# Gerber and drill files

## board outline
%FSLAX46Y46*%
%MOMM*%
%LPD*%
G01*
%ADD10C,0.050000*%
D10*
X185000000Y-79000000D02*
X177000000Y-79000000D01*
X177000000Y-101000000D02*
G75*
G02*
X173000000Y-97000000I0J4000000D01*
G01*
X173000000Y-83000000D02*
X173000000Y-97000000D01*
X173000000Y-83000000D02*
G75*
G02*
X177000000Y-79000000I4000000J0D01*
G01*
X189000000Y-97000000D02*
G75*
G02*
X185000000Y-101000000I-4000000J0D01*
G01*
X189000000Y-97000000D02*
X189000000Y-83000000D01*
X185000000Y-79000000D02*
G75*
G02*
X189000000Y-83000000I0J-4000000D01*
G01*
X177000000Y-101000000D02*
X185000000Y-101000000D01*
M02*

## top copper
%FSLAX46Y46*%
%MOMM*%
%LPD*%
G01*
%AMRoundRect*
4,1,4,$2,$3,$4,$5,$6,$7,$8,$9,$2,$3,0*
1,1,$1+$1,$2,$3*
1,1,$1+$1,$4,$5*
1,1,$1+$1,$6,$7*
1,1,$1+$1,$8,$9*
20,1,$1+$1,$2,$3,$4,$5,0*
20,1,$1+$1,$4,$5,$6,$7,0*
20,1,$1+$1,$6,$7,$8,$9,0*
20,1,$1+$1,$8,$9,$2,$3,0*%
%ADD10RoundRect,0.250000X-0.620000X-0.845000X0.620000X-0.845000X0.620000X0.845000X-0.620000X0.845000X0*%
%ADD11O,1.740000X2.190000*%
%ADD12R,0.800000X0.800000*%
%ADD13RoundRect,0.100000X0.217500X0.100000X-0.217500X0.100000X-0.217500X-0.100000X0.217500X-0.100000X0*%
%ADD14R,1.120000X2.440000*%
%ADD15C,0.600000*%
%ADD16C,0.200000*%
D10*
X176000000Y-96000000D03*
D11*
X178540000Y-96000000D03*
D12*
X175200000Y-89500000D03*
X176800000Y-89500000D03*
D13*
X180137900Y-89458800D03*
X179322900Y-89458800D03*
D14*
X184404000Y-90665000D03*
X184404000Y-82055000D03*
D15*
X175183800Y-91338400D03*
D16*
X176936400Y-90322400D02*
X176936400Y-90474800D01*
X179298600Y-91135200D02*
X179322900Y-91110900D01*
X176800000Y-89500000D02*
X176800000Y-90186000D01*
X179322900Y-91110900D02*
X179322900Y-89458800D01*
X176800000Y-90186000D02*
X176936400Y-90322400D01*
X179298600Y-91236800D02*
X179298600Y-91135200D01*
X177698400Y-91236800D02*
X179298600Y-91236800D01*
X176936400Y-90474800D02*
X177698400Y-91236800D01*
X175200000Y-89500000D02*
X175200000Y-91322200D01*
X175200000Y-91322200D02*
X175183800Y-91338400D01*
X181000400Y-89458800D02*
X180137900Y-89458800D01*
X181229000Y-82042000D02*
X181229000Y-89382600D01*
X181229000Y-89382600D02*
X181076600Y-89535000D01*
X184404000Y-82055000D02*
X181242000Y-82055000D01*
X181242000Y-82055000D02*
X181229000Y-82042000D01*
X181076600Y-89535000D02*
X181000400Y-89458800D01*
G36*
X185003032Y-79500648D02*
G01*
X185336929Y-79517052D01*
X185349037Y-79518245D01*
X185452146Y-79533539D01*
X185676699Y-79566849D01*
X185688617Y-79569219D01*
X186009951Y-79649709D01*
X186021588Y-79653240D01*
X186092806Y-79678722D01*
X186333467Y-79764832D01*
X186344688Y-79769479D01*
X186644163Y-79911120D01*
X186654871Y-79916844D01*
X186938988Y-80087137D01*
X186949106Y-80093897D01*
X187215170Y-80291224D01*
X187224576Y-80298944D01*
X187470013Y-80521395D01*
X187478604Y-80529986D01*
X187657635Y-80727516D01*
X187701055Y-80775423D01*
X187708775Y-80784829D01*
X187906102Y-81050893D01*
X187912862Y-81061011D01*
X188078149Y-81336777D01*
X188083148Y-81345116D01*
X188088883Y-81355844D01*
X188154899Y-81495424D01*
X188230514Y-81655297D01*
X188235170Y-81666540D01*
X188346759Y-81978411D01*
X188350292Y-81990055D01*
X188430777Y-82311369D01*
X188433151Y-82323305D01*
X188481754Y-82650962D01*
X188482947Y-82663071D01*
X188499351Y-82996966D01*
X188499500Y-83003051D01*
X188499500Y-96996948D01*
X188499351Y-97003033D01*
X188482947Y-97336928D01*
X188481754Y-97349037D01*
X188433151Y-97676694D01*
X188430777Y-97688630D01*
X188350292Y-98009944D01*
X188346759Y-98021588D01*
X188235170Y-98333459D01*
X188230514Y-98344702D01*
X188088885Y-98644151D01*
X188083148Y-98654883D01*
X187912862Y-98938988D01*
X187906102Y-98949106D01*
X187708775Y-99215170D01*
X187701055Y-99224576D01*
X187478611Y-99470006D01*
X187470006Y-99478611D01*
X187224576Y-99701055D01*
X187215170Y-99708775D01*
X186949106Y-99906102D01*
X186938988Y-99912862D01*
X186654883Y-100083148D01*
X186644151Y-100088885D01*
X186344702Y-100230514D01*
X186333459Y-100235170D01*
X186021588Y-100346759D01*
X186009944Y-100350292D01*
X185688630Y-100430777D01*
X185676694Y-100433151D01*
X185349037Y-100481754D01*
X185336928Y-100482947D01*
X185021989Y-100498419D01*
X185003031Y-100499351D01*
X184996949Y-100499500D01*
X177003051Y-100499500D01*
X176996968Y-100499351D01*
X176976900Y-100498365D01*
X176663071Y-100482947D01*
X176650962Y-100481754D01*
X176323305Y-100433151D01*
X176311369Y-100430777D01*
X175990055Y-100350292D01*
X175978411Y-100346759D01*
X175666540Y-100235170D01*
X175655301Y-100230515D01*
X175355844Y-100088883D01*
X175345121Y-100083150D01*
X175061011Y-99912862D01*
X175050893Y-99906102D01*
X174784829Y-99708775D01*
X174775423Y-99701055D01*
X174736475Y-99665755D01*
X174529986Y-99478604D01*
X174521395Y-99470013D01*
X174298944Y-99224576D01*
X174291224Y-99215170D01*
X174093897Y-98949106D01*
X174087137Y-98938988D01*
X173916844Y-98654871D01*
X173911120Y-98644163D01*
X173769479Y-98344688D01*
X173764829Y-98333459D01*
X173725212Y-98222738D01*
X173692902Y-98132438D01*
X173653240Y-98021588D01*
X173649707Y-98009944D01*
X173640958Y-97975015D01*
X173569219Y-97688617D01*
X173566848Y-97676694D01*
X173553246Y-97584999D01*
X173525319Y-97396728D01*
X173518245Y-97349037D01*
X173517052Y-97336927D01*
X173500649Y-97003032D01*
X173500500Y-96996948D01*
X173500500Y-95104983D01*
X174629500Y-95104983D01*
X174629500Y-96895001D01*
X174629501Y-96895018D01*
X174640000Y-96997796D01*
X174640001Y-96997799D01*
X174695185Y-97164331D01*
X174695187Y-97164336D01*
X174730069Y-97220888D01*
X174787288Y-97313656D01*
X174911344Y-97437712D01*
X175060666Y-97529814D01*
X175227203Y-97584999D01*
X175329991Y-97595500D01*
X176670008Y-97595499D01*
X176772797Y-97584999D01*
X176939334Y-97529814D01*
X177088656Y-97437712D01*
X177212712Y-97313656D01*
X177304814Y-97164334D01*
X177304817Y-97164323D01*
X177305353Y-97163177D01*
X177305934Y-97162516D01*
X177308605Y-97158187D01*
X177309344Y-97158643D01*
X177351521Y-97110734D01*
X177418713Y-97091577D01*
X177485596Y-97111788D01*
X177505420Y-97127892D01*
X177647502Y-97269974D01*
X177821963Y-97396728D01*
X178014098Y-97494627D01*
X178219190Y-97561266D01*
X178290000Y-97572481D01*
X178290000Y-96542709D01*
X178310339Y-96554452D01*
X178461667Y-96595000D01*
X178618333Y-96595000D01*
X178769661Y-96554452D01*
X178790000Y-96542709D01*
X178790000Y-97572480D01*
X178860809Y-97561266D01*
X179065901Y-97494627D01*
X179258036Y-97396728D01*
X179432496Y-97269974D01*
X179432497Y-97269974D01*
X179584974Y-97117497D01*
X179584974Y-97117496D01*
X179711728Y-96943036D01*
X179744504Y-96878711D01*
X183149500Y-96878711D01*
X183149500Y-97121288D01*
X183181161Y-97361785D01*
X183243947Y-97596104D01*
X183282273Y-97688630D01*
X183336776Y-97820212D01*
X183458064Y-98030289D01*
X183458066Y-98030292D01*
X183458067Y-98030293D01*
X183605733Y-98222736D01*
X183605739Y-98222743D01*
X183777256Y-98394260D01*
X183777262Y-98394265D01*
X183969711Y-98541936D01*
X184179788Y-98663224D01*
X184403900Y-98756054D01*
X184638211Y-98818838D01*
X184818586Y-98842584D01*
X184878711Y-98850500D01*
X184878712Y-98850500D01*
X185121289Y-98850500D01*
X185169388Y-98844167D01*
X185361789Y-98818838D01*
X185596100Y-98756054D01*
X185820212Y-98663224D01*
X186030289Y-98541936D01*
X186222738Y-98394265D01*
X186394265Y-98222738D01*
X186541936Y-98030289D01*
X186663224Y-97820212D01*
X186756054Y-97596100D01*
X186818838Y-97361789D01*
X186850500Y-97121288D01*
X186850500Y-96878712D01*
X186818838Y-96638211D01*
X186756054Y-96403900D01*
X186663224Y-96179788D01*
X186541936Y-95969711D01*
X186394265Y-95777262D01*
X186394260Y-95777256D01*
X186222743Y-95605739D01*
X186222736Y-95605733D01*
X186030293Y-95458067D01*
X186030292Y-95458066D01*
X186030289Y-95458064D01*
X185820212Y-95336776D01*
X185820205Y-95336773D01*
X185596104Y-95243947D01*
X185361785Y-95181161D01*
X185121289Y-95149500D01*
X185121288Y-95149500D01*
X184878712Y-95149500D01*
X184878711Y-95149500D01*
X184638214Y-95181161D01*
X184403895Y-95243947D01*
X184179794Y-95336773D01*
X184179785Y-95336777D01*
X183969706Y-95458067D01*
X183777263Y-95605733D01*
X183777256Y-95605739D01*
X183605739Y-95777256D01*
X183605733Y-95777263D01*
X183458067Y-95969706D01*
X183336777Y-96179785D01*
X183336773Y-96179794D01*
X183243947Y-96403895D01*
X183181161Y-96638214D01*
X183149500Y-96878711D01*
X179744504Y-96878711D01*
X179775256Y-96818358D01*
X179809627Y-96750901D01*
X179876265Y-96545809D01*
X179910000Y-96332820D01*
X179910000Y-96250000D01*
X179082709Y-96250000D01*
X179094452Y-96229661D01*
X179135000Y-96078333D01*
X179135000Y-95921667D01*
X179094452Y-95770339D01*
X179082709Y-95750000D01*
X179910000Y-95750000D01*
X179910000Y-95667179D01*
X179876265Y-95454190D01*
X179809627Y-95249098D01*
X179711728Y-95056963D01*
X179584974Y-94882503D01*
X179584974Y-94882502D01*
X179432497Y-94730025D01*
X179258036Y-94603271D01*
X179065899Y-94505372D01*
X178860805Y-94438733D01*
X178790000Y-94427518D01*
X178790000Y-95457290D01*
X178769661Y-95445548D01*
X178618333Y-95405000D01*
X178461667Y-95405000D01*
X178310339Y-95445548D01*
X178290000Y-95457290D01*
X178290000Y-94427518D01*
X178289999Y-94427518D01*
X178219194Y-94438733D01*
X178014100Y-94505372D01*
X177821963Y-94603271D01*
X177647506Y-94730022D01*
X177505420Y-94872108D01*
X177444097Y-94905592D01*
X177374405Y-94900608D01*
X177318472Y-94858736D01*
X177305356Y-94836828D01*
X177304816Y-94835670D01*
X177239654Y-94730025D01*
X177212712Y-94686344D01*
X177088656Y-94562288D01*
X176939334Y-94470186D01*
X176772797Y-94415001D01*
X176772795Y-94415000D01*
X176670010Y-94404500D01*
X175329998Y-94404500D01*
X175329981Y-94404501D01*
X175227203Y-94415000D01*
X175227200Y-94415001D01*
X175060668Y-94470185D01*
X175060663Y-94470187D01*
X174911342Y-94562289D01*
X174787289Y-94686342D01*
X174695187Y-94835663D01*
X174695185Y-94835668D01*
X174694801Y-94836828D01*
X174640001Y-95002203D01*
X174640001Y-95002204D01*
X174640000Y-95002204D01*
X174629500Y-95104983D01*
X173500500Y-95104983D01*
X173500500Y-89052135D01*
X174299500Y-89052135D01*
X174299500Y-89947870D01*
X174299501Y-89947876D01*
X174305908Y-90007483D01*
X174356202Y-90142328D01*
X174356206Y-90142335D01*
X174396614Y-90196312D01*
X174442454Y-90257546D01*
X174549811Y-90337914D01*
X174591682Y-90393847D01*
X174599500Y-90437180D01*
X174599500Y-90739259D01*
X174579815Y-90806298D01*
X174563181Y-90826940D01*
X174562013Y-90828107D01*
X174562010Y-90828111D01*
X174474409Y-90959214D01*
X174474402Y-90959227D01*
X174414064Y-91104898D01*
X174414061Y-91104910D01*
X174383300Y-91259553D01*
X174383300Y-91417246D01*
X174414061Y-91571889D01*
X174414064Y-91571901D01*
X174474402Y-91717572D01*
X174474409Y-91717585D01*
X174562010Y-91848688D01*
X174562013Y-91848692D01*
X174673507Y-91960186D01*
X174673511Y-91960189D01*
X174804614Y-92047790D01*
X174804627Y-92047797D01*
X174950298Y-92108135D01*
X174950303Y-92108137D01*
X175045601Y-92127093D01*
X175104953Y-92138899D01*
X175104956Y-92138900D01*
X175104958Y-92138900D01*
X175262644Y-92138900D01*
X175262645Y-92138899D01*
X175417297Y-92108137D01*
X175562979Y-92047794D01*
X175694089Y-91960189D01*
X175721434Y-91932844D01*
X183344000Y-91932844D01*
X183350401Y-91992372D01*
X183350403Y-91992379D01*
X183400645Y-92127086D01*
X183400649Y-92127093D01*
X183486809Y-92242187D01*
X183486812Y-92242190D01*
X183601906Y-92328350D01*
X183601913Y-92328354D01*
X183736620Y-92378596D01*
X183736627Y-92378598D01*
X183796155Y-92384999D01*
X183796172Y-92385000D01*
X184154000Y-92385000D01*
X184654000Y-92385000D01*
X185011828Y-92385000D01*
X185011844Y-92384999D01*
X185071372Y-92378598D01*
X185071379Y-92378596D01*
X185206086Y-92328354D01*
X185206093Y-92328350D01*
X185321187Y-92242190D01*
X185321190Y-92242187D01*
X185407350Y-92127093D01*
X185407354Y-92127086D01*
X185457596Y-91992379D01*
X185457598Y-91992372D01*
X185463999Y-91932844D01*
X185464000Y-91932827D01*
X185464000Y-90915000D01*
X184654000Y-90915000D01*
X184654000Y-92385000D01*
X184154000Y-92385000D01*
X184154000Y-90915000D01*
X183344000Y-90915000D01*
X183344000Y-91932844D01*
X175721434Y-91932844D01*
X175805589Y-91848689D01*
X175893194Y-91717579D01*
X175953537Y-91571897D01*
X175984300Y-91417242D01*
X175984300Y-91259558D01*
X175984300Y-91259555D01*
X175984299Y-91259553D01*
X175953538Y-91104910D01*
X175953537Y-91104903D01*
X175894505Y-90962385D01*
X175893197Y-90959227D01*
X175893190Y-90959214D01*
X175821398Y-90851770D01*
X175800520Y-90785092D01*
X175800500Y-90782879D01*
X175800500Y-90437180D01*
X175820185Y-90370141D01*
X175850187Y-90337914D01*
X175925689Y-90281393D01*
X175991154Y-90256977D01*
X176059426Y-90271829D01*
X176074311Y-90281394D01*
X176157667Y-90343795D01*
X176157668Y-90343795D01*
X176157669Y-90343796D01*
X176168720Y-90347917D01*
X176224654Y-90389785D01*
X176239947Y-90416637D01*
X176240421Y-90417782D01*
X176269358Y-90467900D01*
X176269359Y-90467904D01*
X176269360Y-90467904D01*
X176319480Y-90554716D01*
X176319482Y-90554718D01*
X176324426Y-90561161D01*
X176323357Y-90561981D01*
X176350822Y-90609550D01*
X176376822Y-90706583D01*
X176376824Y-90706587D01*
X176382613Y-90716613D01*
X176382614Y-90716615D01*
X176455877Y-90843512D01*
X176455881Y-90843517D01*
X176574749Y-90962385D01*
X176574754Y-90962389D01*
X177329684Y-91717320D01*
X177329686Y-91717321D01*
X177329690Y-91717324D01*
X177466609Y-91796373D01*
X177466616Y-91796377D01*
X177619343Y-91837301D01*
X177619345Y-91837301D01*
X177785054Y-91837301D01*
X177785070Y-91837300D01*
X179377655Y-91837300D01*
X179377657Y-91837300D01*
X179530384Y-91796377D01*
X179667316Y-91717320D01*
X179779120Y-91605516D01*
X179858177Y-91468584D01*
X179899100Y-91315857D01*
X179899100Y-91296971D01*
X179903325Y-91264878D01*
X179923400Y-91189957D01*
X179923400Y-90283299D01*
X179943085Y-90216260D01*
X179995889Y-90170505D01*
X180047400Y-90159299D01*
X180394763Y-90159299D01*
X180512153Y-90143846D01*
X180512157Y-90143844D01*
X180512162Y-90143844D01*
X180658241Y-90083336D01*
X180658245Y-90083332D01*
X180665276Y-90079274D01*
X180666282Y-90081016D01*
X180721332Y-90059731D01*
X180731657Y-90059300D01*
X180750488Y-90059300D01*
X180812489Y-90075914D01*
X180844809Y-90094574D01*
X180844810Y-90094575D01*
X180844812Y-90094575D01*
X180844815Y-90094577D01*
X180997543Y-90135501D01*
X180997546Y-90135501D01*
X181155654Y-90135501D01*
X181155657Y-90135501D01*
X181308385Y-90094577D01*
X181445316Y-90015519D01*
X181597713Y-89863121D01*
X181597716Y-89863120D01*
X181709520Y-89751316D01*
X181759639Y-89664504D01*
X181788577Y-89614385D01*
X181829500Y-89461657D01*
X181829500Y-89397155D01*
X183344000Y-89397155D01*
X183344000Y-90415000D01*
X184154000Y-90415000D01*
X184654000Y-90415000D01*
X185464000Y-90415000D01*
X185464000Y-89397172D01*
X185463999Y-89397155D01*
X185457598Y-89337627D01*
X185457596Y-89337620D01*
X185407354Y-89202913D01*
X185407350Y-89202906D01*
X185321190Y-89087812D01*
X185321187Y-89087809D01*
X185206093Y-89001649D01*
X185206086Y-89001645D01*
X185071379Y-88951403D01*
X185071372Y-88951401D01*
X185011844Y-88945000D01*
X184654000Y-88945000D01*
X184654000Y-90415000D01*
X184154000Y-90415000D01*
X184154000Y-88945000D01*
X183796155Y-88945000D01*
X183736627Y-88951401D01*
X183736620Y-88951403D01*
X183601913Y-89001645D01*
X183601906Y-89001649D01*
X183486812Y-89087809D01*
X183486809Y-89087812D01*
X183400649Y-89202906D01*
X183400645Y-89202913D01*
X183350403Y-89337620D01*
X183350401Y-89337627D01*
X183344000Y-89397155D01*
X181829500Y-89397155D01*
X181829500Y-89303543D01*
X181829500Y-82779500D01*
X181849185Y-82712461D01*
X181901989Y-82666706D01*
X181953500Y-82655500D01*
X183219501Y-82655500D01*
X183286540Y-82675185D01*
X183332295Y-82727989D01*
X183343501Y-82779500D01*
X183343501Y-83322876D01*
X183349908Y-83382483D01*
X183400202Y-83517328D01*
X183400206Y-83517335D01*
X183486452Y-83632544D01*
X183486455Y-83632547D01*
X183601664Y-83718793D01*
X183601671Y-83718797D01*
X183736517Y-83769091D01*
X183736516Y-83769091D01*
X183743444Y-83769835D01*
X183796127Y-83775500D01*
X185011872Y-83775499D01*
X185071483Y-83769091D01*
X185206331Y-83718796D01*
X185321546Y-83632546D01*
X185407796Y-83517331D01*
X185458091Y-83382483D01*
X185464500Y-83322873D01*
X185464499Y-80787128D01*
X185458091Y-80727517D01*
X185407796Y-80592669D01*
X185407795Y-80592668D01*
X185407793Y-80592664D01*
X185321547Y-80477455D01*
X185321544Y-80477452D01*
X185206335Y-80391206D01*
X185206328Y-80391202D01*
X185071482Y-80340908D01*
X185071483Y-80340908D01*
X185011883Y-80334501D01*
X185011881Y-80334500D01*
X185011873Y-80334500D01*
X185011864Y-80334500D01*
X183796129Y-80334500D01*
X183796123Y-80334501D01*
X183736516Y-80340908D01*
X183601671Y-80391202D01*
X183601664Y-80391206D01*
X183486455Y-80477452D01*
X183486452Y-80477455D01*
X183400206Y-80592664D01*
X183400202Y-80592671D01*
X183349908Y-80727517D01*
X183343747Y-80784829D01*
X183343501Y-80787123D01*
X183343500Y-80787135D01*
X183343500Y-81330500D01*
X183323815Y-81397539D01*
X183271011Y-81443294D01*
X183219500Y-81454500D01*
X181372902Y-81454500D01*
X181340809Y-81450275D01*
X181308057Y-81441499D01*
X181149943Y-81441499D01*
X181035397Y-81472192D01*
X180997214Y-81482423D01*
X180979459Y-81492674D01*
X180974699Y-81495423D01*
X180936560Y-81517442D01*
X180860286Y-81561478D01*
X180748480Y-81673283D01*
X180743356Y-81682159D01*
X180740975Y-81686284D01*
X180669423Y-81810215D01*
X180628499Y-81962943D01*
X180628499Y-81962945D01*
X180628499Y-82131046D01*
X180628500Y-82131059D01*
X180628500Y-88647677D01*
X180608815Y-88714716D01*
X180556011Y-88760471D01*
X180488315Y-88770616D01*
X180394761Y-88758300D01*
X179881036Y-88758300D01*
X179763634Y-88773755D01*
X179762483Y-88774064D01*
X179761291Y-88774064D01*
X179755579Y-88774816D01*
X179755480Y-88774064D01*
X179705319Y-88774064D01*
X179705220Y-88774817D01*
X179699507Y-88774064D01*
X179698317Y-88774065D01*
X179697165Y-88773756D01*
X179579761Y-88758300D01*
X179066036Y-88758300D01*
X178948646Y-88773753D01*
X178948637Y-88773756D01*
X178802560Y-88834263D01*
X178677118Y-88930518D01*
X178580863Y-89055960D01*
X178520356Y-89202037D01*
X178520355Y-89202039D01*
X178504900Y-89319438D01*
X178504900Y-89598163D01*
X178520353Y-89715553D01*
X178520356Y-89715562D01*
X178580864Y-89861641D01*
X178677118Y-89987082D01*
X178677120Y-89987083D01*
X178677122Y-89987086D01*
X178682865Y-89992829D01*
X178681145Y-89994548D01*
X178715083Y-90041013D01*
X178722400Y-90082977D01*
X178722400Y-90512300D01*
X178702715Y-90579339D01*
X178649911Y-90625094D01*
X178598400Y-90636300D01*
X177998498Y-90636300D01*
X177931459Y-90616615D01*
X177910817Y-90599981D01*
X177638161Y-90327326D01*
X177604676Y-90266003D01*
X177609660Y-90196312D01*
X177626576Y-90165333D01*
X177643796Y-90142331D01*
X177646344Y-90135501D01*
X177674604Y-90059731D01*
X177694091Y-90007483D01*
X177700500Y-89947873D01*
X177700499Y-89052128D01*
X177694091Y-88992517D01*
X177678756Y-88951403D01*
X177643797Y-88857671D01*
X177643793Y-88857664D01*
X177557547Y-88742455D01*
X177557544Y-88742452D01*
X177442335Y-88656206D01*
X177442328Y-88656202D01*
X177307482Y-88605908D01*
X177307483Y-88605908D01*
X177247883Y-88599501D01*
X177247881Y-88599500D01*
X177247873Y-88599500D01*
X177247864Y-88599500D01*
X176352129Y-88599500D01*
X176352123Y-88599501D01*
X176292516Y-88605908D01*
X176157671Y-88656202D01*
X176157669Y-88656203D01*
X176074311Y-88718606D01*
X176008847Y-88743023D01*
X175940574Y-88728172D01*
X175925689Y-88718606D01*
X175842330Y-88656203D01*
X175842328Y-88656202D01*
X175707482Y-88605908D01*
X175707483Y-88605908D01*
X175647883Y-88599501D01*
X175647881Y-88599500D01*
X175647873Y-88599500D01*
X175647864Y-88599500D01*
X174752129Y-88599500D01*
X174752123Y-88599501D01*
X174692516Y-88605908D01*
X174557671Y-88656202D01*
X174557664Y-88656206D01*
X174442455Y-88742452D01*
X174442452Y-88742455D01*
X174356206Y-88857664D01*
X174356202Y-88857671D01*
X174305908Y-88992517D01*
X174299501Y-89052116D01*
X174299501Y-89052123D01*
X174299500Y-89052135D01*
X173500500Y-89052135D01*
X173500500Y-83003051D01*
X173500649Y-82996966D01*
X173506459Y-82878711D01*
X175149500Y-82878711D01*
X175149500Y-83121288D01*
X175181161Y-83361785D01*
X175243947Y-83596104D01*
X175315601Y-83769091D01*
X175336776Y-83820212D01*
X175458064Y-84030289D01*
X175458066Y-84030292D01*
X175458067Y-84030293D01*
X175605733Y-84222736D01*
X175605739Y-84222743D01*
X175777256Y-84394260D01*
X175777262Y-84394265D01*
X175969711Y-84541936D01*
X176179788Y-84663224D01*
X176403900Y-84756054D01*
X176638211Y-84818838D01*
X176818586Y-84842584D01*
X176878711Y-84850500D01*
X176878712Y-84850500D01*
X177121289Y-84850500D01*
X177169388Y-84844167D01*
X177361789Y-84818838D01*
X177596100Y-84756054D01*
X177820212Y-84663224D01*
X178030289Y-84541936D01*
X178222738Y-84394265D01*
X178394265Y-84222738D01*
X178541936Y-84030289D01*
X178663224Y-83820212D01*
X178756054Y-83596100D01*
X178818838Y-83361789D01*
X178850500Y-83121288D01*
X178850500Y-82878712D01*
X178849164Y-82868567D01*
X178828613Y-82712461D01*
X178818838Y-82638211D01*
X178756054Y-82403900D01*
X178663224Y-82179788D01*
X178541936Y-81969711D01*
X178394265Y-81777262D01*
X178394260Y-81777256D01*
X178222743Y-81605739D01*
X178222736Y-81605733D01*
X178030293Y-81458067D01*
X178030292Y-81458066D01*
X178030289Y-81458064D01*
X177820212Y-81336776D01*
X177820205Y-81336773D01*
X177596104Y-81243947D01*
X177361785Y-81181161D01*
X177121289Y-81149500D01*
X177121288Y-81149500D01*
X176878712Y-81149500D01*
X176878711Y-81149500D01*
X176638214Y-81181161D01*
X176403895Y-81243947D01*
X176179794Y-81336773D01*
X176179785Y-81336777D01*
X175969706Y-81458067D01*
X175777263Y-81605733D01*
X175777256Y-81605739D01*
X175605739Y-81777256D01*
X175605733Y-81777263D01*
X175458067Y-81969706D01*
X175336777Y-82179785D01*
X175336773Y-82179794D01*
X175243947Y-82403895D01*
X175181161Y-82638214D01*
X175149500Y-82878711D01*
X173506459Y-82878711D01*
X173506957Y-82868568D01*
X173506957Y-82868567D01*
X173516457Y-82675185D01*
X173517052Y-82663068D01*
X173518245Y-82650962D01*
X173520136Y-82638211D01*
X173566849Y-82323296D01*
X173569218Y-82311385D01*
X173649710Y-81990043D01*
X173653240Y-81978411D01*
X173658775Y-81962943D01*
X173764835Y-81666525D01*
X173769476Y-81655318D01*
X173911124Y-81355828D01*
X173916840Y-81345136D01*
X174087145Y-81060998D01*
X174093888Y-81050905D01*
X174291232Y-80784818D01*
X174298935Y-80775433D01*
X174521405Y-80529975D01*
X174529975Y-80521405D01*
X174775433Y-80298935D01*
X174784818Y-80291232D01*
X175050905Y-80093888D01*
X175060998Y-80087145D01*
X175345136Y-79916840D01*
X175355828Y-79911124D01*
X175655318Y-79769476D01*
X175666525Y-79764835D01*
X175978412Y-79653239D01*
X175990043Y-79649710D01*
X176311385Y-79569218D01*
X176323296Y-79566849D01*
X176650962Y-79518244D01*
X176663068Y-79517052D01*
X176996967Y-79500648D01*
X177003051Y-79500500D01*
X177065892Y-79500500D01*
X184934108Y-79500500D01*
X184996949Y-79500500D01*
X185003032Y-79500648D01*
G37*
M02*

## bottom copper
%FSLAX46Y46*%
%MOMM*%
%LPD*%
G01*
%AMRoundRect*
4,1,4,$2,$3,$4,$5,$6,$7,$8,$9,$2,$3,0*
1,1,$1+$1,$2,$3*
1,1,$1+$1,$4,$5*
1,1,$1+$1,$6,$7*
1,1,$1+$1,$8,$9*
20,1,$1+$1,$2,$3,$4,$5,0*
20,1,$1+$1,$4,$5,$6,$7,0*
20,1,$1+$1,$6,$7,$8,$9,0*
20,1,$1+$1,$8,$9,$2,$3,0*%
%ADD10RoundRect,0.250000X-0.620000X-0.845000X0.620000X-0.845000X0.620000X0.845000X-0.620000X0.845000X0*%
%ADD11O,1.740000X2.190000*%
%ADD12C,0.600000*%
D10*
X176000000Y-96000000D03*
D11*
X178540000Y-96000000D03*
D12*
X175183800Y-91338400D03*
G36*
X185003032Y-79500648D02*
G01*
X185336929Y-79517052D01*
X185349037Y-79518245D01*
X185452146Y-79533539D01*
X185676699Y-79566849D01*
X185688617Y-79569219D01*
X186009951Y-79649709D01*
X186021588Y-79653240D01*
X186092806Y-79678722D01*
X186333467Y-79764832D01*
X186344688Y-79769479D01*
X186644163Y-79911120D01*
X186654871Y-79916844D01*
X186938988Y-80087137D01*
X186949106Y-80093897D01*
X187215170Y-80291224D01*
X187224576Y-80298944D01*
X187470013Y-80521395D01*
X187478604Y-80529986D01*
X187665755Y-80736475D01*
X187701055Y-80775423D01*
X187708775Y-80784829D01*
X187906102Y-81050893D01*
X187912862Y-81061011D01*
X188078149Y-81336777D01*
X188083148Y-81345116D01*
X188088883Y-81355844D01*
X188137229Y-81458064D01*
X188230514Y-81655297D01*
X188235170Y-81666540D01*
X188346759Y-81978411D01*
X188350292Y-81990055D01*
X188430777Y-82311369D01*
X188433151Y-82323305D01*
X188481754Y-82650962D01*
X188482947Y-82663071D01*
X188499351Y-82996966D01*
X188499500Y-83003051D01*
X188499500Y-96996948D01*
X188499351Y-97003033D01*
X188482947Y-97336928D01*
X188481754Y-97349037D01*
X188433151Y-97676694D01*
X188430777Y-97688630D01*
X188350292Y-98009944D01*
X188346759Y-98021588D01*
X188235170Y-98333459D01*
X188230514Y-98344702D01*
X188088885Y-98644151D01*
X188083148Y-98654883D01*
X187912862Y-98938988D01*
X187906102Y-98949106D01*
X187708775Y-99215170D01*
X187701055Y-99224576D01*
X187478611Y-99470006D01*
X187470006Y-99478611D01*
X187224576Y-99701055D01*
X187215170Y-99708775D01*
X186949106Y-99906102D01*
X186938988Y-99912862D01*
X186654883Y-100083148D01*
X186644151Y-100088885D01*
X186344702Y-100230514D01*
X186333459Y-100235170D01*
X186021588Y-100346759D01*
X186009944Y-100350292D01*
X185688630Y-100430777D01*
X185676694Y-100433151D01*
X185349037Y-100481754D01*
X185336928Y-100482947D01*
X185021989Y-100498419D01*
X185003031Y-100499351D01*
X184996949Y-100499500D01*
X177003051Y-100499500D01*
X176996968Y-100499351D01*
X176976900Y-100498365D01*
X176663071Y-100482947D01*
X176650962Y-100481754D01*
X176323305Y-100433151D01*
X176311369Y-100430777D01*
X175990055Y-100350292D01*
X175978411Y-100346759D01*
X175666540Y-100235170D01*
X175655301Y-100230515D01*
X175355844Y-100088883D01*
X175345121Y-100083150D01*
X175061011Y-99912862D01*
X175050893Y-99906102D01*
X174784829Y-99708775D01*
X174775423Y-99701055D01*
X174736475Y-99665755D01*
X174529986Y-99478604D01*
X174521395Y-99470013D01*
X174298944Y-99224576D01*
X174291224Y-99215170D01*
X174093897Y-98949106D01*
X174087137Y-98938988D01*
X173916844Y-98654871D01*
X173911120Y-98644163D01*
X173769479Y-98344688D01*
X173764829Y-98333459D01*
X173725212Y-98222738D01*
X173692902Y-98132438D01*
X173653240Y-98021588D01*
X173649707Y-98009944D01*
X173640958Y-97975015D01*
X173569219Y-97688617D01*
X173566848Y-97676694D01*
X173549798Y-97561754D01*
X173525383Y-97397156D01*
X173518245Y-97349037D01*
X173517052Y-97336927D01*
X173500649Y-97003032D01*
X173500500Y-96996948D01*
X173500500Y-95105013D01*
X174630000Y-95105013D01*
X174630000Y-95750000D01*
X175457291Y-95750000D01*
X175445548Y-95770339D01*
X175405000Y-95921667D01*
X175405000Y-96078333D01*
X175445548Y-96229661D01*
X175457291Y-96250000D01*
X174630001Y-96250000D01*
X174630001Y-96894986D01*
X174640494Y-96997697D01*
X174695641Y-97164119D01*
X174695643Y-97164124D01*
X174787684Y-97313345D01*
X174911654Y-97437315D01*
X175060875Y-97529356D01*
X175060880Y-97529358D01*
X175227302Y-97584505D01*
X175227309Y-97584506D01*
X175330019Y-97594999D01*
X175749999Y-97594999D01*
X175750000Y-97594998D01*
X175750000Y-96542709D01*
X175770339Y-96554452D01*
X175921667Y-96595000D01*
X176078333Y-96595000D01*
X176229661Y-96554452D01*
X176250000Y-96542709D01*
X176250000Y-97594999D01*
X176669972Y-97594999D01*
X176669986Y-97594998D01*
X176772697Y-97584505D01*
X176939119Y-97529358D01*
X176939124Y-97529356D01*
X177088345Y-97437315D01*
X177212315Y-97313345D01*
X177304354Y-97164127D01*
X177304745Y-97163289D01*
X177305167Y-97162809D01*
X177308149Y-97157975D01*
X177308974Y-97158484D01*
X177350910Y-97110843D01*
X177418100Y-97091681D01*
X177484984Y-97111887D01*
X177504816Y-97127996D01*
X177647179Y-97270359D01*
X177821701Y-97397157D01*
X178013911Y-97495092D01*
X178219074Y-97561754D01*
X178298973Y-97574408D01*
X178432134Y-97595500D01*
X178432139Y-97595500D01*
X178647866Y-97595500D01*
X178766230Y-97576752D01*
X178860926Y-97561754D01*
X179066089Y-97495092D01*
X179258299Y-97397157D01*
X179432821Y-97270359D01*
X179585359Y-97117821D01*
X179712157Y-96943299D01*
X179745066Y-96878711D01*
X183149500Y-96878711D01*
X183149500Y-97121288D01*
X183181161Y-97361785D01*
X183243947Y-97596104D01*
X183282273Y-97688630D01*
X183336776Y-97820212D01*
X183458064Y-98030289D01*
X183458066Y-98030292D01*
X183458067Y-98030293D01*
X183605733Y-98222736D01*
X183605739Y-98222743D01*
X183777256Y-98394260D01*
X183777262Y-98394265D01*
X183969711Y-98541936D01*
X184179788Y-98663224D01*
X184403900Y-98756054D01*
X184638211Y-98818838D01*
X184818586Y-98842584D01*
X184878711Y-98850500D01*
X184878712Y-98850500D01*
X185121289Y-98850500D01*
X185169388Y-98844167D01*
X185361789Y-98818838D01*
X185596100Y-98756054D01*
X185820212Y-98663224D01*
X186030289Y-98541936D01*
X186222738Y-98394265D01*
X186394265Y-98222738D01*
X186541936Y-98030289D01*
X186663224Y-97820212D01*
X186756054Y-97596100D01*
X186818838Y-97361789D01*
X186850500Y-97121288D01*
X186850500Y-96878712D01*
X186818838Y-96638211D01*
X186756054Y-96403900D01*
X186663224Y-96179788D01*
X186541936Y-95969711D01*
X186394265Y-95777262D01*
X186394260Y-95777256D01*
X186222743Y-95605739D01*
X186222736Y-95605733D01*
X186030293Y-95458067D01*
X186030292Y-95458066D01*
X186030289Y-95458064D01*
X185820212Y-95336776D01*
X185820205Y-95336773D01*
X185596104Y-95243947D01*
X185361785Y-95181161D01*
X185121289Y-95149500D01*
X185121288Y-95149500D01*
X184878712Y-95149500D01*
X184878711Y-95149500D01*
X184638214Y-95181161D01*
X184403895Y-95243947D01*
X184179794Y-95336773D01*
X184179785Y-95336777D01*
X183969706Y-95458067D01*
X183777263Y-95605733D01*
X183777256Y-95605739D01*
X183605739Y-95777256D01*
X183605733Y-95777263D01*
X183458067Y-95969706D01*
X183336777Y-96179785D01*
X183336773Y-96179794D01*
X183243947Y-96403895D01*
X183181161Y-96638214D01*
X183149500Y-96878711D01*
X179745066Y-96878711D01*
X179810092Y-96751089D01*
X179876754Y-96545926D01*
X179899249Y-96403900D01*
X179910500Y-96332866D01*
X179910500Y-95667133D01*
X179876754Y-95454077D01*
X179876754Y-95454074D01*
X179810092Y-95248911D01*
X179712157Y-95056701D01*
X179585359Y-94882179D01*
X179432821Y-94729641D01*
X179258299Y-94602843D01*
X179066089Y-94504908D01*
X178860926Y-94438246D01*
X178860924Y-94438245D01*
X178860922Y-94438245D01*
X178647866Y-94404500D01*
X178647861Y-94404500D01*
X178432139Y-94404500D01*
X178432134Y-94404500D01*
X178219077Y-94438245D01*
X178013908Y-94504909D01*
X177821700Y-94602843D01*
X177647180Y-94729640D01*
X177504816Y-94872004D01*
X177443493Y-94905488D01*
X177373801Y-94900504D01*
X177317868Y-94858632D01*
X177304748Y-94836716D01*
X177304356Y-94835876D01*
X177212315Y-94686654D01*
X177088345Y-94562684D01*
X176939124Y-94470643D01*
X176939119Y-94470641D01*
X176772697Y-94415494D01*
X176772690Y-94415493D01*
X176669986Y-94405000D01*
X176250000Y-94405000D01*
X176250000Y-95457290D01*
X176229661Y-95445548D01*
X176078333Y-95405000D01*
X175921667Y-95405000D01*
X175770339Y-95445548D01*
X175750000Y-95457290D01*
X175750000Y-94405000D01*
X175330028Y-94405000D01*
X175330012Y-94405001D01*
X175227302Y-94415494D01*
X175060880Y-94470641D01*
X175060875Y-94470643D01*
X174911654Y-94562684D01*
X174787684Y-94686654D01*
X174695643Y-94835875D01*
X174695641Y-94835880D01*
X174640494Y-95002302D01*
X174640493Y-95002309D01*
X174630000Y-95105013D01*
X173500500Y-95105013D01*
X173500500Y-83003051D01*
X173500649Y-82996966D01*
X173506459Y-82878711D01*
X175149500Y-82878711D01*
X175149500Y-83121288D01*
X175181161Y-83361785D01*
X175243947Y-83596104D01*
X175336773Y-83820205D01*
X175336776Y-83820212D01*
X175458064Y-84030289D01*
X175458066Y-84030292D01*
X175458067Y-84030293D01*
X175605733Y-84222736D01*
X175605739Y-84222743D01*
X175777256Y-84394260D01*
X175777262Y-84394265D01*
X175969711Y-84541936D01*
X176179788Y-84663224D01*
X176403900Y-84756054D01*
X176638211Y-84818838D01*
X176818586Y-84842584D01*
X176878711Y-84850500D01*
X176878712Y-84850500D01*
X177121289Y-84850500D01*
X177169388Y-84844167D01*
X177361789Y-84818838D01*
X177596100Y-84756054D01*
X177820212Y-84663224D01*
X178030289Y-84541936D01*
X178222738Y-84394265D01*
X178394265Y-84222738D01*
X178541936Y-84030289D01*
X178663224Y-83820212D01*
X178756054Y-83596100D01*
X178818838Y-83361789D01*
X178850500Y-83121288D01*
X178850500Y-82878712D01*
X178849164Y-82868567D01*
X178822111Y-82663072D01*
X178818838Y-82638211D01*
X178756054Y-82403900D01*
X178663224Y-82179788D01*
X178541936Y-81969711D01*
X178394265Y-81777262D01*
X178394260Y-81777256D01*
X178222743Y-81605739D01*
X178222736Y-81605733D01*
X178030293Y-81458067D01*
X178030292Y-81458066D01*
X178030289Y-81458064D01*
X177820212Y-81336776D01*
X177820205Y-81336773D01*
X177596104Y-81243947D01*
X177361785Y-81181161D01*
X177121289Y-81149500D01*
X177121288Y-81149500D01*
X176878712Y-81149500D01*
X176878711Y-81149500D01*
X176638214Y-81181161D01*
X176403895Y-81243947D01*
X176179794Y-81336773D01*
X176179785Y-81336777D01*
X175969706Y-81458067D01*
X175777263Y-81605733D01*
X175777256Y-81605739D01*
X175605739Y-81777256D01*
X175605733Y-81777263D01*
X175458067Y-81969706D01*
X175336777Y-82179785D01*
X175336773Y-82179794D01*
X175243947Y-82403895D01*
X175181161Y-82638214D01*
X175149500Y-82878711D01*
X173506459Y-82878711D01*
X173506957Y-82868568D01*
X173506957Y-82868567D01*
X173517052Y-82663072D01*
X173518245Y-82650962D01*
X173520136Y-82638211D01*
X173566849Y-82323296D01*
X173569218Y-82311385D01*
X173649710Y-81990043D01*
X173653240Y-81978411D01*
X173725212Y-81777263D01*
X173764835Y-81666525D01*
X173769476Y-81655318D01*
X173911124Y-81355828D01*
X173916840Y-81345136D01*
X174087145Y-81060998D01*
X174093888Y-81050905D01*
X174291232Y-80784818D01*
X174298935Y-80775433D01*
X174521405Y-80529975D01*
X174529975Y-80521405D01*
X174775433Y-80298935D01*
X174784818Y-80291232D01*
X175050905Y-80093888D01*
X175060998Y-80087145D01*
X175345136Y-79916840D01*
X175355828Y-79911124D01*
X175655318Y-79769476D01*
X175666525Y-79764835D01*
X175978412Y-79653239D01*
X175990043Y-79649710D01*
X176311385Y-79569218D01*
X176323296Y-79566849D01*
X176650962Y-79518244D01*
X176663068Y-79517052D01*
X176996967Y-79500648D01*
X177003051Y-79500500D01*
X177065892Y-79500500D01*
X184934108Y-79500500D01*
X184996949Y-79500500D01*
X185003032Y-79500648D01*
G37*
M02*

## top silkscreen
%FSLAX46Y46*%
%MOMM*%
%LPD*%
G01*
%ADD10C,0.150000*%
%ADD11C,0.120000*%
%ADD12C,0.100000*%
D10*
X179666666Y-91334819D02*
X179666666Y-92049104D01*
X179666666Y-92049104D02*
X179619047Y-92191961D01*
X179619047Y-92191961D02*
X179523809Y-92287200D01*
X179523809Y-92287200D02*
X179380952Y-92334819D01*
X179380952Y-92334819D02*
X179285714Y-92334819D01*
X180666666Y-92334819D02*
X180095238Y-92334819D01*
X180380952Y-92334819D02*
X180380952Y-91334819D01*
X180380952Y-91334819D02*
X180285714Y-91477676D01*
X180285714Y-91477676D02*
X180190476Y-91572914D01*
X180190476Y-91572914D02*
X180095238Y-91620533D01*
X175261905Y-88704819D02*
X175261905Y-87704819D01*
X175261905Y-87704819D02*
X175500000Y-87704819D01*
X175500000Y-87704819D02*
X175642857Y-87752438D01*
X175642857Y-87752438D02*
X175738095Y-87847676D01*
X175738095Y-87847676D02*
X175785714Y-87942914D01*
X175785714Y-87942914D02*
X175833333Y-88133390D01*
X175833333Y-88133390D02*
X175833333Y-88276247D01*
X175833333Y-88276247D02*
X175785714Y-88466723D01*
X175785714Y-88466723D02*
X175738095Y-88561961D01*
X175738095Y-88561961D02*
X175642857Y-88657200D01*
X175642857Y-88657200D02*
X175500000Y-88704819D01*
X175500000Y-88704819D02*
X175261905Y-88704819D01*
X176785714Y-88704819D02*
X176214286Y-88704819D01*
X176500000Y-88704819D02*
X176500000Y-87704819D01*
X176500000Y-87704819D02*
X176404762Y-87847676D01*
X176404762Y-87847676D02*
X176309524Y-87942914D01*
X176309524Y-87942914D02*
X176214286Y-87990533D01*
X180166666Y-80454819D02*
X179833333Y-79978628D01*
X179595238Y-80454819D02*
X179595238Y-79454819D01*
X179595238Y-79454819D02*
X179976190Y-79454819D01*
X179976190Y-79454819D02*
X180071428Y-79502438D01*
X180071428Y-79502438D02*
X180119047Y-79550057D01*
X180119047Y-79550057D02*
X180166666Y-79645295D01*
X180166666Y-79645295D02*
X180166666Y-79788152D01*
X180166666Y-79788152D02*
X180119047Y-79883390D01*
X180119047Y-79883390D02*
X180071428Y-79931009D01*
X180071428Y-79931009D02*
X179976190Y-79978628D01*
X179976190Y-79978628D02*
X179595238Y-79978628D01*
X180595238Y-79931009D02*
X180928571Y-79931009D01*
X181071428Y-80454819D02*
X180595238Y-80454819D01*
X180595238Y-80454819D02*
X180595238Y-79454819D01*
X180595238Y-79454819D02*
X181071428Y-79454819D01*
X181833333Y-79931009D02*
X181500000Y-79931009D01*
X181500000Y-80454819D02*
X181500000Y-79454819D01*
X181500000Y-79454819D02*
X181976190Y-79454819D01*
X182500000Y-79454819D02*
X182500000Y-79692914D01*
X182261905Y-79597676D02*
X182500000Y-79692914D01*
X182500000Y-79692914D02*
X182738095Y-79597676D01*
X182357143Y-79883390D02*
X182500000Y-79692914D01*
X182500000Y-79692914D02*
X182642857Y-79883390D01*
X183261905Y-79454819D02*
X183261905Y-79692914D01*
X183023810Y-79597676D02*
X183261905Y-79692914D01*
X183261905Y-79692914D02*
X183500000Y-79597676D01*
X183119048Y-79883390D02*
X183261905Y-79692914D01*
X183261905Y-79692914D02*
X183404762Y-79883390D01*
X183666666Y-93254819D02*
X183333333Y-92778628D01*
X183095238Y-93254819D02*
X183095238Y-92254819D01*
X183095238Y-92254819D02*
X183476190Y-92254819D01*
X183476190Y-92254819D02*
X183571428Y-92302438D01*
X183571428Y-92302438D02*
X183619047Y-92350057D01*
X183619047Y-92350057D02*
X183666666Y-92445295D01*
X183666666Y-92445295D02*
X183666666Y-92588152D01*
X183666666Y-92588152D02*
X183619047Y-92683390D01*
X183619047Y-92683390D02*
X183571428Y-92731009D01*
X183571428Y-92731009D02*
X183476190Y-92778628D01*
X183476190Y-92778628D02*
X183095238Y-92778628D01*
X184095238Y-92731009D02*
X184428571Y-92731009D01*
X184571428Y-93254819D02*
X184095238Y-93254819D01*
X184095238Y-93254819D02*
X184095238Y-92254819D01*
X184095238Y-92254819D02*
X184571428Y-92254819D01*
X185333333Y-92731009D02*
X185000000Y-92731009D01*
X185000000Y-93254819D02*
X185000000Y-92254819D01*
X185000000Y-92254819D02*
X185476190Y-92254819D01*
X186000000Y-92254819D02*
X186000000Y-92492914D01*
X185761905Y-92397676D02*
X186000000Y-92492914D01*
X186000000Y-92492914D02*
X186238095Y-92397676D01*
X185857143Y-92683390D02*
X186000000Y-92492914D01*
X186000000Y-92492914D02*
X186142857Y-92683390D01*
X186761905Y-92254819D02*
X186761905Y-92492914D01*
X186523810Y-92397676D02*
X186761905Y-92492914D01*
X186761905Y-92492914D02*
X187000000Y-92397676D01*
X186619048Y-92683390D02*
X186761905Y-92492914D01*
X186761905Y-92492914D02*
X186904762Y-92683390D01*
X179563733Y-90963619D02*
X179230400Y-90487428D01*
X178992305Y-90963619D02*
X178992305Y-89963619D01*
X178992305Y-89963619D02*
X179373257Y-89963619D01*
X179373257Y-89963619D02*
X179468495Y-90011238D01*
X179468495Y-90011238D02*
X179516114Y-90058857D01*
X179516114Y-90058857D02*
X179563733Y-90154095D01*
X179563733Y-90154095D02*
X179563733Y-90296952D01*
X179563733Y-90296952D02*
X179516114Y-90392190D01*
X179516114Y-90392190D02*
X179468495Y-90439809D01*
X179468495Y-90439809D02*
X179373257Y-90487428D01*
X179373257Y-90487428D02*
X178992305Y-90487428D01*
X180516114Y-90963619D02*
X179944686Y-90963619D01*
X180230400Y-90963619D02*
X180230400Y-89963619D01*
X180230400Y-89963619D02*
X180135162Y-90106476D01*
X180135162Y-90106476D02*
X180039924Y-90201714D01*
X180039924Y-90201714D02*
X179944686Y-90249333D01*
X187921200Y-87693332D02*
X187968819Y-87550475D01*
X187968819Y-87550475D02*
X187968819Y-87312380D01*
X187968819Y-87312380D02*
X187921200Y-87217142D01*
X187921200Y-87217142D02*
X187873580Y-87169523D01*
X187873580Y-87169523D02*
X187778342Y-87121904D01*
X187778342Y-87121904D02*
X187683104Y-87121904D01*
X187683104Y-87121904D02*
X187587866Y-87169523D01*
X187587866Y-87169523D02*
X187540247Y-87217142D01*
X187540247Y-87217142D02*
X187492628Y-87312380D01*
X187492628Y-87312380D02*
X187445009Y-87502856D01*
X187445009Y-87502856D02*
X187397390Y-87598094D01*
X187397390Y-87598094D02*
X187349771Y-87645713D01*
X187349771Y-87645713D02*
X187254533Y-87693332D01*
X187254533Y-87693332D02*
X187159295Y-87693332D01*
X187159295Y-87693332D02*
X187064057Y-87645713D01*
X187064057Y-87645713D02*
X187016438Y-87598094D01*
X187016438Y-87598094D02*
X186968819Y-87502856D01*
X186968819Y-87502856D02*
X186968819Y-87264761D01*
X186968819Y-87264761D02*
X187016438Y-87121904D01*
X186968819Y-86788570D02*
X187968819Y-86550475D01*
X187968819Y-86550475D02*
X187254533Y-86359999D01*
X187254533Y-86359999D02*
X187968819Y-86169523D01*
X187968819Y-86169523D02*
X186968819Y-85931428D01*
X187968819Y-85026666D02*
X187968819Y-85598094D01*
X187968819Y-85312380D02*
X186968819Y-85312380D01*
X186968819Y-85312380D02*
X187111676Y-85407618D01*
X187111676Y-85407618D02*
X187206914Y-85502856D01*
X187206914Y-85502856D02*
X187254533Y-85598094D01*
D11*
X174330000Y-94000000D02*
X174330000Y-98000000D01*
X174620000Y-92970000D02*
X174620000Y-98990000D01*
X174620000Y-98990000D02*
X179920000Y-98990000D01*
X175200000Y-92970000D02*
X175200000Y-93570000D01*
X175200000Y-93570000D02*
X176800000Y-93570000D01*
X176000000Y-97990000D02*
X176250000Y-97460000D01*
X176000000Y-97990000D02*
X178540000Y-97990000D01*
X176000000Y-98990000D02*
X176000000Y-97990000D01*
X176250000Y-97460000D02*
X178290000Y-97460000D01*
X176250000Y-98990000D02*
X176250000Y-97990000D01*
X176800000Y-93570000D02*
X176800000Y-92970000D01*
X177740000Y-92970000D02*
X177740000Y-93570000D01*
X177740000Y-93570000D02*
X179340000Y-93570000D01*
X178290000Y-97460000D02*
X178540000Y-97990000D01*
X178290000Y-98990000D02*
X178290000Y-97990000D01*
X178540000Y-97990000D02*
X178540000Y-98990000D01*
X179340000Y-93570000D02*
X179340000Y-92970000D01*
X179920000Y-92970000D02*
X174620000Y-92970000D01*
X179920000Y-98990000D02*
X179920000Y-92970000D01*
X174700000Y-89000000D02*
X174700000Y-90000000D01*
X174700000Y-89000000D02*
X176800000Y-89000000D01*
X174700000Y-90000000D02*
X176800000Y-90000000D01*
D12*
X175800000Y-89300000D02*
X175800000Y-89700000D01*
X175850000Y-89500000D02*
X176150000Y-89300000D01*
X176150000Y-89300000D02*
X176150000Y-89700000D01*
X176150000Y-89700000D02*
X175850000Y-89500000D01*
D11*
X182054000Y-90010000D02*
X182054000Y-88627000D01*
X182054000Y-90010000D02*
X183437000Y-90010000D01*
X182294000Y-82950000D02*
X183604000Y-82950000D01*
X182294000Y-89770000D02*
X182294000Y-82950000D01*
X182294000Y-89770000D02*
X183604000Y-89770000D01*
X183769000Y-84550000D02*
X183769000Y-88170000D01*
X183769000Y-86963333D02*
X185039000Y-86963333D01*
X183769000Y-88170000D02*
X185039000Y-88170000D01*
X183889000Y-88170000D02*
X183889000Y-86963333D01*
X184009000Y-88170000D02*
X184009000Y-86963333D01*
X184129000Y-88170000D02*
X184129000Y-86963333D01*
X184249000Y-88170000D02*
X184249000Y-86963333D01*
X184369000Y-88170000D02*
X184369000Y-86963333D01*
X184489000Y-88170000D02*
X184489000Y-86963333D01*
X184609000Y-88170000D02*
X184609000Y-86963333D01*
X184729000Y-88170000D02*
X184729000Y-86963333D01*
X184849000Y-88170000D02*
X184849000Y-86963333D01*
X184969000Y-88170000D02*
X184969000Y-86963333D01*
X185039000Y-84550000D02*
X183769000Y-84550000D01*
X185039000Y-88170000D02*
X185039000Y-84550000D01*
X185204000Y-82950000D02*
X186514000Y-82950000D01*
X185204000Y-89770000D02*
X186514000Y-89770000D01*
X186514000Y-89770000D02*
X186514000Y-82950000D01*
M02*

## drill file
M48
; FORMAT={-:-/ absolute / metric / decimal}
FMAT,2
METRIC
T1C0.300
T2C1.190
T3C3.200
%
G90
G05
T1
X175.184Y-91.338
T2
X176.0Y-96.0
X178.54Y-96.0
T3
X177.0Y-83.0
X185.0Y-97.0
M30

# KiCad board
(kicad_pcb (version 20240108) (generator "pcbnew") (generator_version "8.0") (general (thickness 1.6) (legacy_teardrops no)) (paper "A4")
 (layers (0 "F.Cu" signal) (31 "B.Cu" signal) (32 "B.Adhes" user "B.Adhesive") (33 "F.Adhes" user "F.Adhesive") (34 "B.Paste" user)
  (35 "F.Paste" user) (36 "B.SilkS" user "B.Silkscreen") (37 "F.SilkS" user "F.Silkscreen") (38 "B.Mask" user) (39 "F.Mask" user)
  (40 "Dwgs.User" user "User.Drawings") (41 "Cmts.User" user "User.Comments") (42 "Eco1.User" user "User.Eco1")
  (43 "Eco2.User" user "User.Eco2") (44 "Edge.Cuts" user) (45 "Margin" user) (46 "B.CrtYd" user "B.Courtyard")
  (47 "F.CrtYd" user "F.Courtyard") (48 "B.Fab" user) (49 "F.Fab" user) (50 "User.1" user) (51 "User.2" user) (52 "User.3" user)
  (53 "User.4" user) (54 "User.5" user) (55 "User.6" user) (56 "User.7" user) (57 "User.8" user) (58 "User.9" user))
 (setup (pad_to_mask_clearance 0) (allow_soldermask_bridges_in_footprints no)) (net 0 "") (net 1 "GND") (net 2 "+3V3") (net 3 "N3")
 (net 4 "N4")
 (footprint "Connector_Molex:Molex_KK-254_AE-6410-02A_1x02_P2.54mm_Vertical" (layer "F.Cu") (at 176 96)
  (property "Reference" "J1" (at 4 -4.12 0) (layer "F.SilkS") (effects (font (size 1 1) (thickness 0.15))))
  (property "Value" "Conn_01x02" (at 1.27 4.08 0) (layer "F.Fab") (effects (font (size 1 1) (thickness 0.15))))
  (fp_line (start -1.67 -2) (end -1.67 2) (stroke (width 0.12) (type solid)) (layer "F.SilkS"))
  (fp_line (start -1.38 -3.03) (end -1.38 2.99) (stroke (width 0.12) (type solid)) (layer "F.SilkS"))
  (fp_line (start -1.38 2.99) (end 3.92 2.99) (stroke (width 0.12) (type solid)) (layer "F.SilkS"))
  (fp_line (start -0.8 -3.03) (end -0.8 -2.43) (stroke (width 0.12) (type solid)) (layer "F.SilkS"))
  (fp_line (start -0.8 -2.43) (end 0.8 -2.43) (stroke (width 0.12) (type solid)) (layer "F.SilkS"))
  (fp_line (start 0 1.99) (end 0.25 1.46) (stroke (width 0.12) (type solid)) (layer "F.SilkS"))
  (fp_line (start 0 1.99) (end 2.54 1.99) (stroke (width 0.12) (type solid)) (layer "F.SilkS"))
  (fp_line (start 0 2.99) (end 0 1.99) (stroke (width 0.12) (type solid)) (layer "F.SilkS"))
  (fp_line (start 0.25 1.46) (end 2.29 1.46) (stroke (width 0.12) (type solid)) (layer "F.SilkS"))
  (fp_line (start 0.25 2.99) (end 0.25 1.99) (stroke (width 0.12) (type solid)) (layer "F.SilkS"))
  (fp_line (start 0.8 -2.43) (end 0.8 -3.03) (stroke (width 0.12) (type solid)) (layer "F.SilkS"))
  (fp_line (start 1.74 -3.03) (end 1.74 -2.43) (stroke (width 0.12) (type solid)) (layer "F.SilkS"))
  (fp_line (start 1.74 -2.43) (end 3.34 -2.43) (stroke (width 0.12) (type solid)) (layer "F.SilkS"))
  (fp_line (start 2.29 1.46) (end 2.54 1.99) (stroke (width 0.12) (type solid)) (layer "F.SilkS"))
  (fp_line (start 2.29 2.99) (end 2.29 1.99) (stroke (width 0.12) (type solid)) (layer "F.SilkS"))
  (fp_line (start 2.54 1.99) (end 2.54 2.99) (stroke (width 0.12) (type solid)) (layer "F.SilkS"))
  (fp_line (start 3.34 -2.43) (end 3.34 -3.03) (stroke (width 0.12) (type solid)) (layer "F.SilkS"))
  (fp_line (start 3.92 -3.03) (end -1.38 -3.03) (stroke (width 0.12) (type solid)) (layer "F.SilkS"))
  (fp_line (start 3.92 2.99) (end 3.92 -3.03) (stroke (width 0.12) (type solid)) (layer "F.SilkS"))
  (pad "1" thru_hole roundrect (at 0 0) (size 1.74 2.19) (drill 1.19) (layers "*.Cu" "*.Mask") (remove_unused_layers no)
   (roundrect_rratio 0.143678) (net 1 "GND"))
  (pad "2" thru_hole oval (at 2.54 0) (size 1.74 2.19) (drill 1.19) (layers "*.Cu" "*.Mask") (remove_unused_layers no) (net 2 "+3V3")))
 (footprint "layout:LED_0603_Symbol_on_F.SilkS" (layer "F.Cu") (at 176 89.5)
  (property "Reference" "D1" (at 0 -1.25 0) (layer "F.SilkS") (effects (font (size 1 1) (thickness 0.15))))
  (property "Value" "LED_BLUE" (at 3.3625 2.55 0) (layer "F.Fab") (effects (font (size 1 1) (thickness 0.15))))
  (fp_line (start -1.3 -0.5) (end -1.3 0.5) (stroke (width 0.12) (type solid)) (layer "F.SilkS"))
  (fp_line (start -1.3 -0.5) (end 0.8 -0.5) (stroke (width 0.12) (type solid)) (layer "F.SilkS"))
  (fp_line (start -1.3 0.5) (end 0.8 0.5) (stroke (width 0.12) (type solid)) (layer "F.SilkS"))
  (fp_line (start -0.2 -0.2) (end -0.2 0.2) (stroke (width 0.1) (type solid)) (layer "F.SilkS"))
  (fp_line (start -0.15 0) (end 0.15 -0.2) (stroke (width 0.1) (type solid)) (layer "F.SilkS"))
  (fp_line (start 0.15 -0.2) (end 0.15 0.2) (stroke (width 0.1) (type solid)) (layer "F.SilkS"))
  (fp_line (start 0.15 0.2) (end -0.15 0) (stroke (width 0.1) (type solid)) (layer "F.SilkS"))
  (pad "1" smd rect (at -0.8 0 180) (size 0.8 0.8) (layers "F.Cu" "F.Paste" "F.Mask") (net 1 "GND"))
  (pad "2" smd rect (at 0.8 0 180) (size 0.8 0.8) (layers "F.Cu" "F.Paste" "F.Mask") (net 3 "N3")))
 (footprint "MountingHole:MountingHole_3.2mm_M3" (layer "F.Cu") (at 177 83)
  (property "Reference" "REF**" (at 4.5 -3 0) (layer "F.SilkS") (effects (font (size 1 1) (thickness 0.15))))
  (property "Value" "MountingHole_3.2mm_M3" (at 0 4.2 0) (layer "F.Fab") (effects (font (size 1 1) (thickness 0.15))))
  (pad "" np_thru_hole circle (at 0 0) (size 3.2 3.2) (drill 3.2) (layers "*.Cu" "*.Mask")))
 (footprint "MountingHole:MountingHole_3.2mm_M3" (layer "F.Cu") (at 185 97)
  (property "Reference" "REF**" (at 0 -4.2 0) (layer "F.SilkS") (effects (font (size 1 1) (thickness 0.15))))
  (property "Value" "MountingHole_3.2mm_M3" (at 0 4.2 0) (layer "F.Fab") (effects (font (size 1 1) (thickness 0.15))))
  (pad "" np_thru_hole circle (at 0 0) (size 3.2 3.2) (drill 3.2) (layers "*.Cu" "*.Mask")))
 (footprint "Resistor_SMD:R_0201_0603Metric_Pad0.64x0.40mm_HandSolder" (layer "F.Cu") (at 179.7304 89.4588 180)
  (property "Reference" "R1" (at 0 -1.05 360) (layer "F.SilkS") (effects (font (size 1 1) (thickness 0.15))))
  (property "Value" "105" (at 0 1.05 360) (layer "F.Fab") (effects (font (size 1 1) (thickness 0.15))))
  (pad "" smd roundrect (at -0.4325 0 180) (size 0.458 0.36) (layers "F.Paste") (roundrect_rratio 0.25))
  (pad "" smd roundrect (at 0.4325 0 180) (size 0.458 0.36) (layers "F.Paste") (roundrect_rratio 0.25))
  (pad "1" smd roundrect (at -0.4075 0 180) (size 0.635 0.4) (layers "F.Cu" "F.Mask") (roundrect_rratio 0.25) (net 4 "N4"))
  (pad "2" smd roundrect (at 0.4075 0 180) (size 0.635 0.4) (layers "F.Cu" "F.Mask") (roundrect_rratio 0.25) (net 3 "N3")))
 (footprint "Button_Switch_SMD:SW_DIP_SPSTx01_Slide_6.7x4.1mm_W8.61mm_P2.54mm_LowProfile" (layer "F.Cu") (at 184.404 86.36 90)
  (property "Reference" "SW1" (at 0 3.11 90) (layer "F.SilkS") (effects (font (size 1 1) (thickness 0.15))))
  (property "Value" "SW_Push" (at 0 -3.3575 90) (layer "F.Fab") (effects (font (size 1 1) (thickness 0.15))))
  (fp_line (start -3.65 -2.35) (end -2.267 -2.35) (stroke (width 0.12) (type solid)) (layer "F.SilkS"))
  (fp_line (start -3.65 -2.35) (end -3.65 -0.967) (stroke (width 0.12) (type solid)) (layer "F.SilkS"))
  (fp_line (start 3.41 -2.11) (end 3.41 -0.8) (stroke (width 0.12) (type solid)) (layer "F.SilkS"))
  (fp_line (start -3.41 -2.11) (end 3.41 -2.11) (stroke (width 0.12) (type solid)) (layer "F.SilkS"))
  (fp_line (start -3.41 -2.11) (end -3.41 -0.8) (stroke (width 0.12) (type solid)) (layer "F.SilkS"))
  (fp_line (start 1.81 -0.635) (end -1.81 -0.635) (stroke (width 0.12) (type solid)) (layer "F.SilkS"))
  (fp_line (start -0.603333 -0.635) (end -0.603333 0.635) (stroke (width 0.12) (type solid)) (layer "F.SilkS"))
  (fp_line (start -1.81 -0.635) (end -1.81 0.635) (stroke (width 0.12) (type solid)) (layer "F.SilkS"))
  (fp_line (start -1.81 -0.515) (end -0.603333 -0.515) (stroke (width 0.12) (type solid)) (layer "F.SilkS"))
  (fp_line (start -1.81 -0.395) (end -0.603333 -0.395) (stroke (width 0.12) (type solid)) (layer "F.SilkS"))
  (fp_line (start -1.81 -0.275) (end -0.603333 -0.275) (stroke (width 0.12) (type solid)) (layer "F.SilkS"))
  (fp_line (start -1.81 -0.155) (end -0.603333 -0.155) (stroke (width 0.12) (type solid)) (layer "F.SilkS"))
  (fp_line (start -1.81 -0.035) (end -0.603333 -0.035) (stroke (width 0.12) (type solid)) (layer "F.SilkS"))
  (fp_line (start -1.81 0.085) (end -0.603333 0.085) (stroke (width 0.12) (type solid)) (layer "F.SilkS"))
  (fp_line (start -1.81 0.205) (end -0.603333 0.205) (stroke (width 0.12) (type solid)) (layer "F.SilkS"))
  (fp_line (start -1.81 0.325) (end -0.603333 0.325) (stroke (width 0.12) (type solid)) (layer "F.SilkS"))
  (fp_line (start -1.81 0.445) (end -0.603333 0.445) (stroke (width 0.12) (type solid)) (layer "F.SilkS"))
  (fp_line (start -1.81 0.565) (end -0.603333 0.565) (stroke (width 0.12) (type solid)) (layer "F.SilkS"))
  (fp_line (start 1.81 0.635) (end 1.81 -0.635) (stroke (width 0.12) (type solid)) (layer "F.SilkS"))
  (fp_line (start -1.81 0.635) (end 1.81 0.635) (stroke (width 0.12) (type solid)) (layer "F.SilkS"))
  (fp_line (start 3.41 0.8) (end 3.41 2.11) (stroke (width 0.12) (type solid)) (layer "F.SilkS"))
  (fp_line (start -3.41 0.8) (end -3.41 2.11) (stroke (width 0.12) (type solid)) (layer "F.SilkS"))
  (fp_line (start -3.41 2.11) (end 3.41 2.11) (stroke (width 0.12) (type solid)) (layer "F.SilkS"))
  (pad "1" smd rect (at -4.305 0 90) (size 2.44 1.12) (layers "F.Cu" "F.Paste" "F.Mask") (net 2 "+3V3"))
  (pad "2" smd rect (at 4.305 0 90) (size 2.44 1.12) (layers "F.Cu" "F.Paste" "F.Mask") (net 4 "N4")))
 (gr_line (start 185 79) (end 177 79) (stroke (width 0.05) (type default)) (layer "Edge.Cuts"))
 (gr_arc (start 177 101) (mid 174.171573 99.828427) (end 173 97) (stroke (width 0.05) (type default)) (layer "Edge.Cuts"))
 (gr_line (start 173 83) (end 173 97) (stroke (width 0.05) (type default)) (layer "Edge.Cuts"))
 (gr_arc (start 173 83) (mid 174.171573 80.171573) (end 177 79) (stroke (width 0.05) (type default)) (layer "Edge.Cuts"))
 (gr_arc (start 189 97) (mid 187.828427 99.828427) (end 185 101) (stroke (width 0.05) (type default)) (layer "Edge.Cuts"))
 (gr_line (start 189 97) (end 189 83) (stroke (width 0.05) (type default)) (layer "Edge.Cuts"))
 (gr_arc (start 185 79) (mid 187.828427 80.171573) (end 189 83) (stroke (width 0.05) (type default)) (layer "Edge.Cuts"))
 (gr_line (start 177 101) (end 185 101) (stroke (width 0.05) (type default)) (layer "Edge.Cuts"))
 (segment (start 176.9364 90.3224) (end 176.9364 90.4748) (width 0.2) (layer "F.Cu") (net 3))
 (segment (start 179.2986 91.1352) (end 179.3229 91.1109) (width 0.2) (layer "F.Cu") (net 3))
 (segment (start 176.8 89.5) (end 176.8 90.186) (width 0.2) (layer "F.Cu") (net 3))
 (segment (start 179.3229 91.1109) (end 179.3229 89.4588) (width 0.2) (layer "F.Cu") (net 3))
 (segment (start 176.8 90.186) (end 176.9364 90.3224) (width 0.2) (layer "F.Cu") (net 3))
 (segment (start 179.2986 91.2368) (end 179.2986 91.1352) (width 0.2) (layer "F.Cu") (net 3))
 (segment (start 177.6984 91.2368) (end 179.2986 91.2368) (width 0.2) (layer "F.Cu") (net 3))
 (segment (start 176.9364 90.4748) (end 177.6984 91.2368) (width 0.2) (layer "F.Cu") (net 3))
 (segment (start 175.2 89.5) (end 175.2 91.3222) (width 0.2) (layer "F.Cu") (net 1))
 (segment (start 175.2 91.3222) (end 175.1838 91.3384) (width 0.2) (layer "F.Cu") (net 1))
 (via (at 175.1838 91.3384) (size 0.6) (drill 0.3) (layers "F.Cu" "B.Cu") (free yes) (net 1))
 (segment (start 181.0004 89.4588) (end 180.1379 89.4588) (width 0.2) (layer "F.Cu") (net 4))
 (segment (start 181.229 82.042) (end 181.229 89.3826) (width 0.2) (layer "F.Cu") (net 4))
 (segment (start 181.229 89.3826) (end 181.0766 89.535) (width 0.2) (layer "F.Cu") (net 4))
 (segment (start 184.404 82.055) (end 181.242 82.055) (width 0.2) (layer "F.Cu") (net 4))
 (segment (start 181.242 82.055) (end 181.229 82.042) (width 0.2) (layer "F.Cu") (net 4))
 (segment (start 181.0766 89.535) (end 181.0004 89.4588) (width 0.2) (layer "F.Cu") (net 4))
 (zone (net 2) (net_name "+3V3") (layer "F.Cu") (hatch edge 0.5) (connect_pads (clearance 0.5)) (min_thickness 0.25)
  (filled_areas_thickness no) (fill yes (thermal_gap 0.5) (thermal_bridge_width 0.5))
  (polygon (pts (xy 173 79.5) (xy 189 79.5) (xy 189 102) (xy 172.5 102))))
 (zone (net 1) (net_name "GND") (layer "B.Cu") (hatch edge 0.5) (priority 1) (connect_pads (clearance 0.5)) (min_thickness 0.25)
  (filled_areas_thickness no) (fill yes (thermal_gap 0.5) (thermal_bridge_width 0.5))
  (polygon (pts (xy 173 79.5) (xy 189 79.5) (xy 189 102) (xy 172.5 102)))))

